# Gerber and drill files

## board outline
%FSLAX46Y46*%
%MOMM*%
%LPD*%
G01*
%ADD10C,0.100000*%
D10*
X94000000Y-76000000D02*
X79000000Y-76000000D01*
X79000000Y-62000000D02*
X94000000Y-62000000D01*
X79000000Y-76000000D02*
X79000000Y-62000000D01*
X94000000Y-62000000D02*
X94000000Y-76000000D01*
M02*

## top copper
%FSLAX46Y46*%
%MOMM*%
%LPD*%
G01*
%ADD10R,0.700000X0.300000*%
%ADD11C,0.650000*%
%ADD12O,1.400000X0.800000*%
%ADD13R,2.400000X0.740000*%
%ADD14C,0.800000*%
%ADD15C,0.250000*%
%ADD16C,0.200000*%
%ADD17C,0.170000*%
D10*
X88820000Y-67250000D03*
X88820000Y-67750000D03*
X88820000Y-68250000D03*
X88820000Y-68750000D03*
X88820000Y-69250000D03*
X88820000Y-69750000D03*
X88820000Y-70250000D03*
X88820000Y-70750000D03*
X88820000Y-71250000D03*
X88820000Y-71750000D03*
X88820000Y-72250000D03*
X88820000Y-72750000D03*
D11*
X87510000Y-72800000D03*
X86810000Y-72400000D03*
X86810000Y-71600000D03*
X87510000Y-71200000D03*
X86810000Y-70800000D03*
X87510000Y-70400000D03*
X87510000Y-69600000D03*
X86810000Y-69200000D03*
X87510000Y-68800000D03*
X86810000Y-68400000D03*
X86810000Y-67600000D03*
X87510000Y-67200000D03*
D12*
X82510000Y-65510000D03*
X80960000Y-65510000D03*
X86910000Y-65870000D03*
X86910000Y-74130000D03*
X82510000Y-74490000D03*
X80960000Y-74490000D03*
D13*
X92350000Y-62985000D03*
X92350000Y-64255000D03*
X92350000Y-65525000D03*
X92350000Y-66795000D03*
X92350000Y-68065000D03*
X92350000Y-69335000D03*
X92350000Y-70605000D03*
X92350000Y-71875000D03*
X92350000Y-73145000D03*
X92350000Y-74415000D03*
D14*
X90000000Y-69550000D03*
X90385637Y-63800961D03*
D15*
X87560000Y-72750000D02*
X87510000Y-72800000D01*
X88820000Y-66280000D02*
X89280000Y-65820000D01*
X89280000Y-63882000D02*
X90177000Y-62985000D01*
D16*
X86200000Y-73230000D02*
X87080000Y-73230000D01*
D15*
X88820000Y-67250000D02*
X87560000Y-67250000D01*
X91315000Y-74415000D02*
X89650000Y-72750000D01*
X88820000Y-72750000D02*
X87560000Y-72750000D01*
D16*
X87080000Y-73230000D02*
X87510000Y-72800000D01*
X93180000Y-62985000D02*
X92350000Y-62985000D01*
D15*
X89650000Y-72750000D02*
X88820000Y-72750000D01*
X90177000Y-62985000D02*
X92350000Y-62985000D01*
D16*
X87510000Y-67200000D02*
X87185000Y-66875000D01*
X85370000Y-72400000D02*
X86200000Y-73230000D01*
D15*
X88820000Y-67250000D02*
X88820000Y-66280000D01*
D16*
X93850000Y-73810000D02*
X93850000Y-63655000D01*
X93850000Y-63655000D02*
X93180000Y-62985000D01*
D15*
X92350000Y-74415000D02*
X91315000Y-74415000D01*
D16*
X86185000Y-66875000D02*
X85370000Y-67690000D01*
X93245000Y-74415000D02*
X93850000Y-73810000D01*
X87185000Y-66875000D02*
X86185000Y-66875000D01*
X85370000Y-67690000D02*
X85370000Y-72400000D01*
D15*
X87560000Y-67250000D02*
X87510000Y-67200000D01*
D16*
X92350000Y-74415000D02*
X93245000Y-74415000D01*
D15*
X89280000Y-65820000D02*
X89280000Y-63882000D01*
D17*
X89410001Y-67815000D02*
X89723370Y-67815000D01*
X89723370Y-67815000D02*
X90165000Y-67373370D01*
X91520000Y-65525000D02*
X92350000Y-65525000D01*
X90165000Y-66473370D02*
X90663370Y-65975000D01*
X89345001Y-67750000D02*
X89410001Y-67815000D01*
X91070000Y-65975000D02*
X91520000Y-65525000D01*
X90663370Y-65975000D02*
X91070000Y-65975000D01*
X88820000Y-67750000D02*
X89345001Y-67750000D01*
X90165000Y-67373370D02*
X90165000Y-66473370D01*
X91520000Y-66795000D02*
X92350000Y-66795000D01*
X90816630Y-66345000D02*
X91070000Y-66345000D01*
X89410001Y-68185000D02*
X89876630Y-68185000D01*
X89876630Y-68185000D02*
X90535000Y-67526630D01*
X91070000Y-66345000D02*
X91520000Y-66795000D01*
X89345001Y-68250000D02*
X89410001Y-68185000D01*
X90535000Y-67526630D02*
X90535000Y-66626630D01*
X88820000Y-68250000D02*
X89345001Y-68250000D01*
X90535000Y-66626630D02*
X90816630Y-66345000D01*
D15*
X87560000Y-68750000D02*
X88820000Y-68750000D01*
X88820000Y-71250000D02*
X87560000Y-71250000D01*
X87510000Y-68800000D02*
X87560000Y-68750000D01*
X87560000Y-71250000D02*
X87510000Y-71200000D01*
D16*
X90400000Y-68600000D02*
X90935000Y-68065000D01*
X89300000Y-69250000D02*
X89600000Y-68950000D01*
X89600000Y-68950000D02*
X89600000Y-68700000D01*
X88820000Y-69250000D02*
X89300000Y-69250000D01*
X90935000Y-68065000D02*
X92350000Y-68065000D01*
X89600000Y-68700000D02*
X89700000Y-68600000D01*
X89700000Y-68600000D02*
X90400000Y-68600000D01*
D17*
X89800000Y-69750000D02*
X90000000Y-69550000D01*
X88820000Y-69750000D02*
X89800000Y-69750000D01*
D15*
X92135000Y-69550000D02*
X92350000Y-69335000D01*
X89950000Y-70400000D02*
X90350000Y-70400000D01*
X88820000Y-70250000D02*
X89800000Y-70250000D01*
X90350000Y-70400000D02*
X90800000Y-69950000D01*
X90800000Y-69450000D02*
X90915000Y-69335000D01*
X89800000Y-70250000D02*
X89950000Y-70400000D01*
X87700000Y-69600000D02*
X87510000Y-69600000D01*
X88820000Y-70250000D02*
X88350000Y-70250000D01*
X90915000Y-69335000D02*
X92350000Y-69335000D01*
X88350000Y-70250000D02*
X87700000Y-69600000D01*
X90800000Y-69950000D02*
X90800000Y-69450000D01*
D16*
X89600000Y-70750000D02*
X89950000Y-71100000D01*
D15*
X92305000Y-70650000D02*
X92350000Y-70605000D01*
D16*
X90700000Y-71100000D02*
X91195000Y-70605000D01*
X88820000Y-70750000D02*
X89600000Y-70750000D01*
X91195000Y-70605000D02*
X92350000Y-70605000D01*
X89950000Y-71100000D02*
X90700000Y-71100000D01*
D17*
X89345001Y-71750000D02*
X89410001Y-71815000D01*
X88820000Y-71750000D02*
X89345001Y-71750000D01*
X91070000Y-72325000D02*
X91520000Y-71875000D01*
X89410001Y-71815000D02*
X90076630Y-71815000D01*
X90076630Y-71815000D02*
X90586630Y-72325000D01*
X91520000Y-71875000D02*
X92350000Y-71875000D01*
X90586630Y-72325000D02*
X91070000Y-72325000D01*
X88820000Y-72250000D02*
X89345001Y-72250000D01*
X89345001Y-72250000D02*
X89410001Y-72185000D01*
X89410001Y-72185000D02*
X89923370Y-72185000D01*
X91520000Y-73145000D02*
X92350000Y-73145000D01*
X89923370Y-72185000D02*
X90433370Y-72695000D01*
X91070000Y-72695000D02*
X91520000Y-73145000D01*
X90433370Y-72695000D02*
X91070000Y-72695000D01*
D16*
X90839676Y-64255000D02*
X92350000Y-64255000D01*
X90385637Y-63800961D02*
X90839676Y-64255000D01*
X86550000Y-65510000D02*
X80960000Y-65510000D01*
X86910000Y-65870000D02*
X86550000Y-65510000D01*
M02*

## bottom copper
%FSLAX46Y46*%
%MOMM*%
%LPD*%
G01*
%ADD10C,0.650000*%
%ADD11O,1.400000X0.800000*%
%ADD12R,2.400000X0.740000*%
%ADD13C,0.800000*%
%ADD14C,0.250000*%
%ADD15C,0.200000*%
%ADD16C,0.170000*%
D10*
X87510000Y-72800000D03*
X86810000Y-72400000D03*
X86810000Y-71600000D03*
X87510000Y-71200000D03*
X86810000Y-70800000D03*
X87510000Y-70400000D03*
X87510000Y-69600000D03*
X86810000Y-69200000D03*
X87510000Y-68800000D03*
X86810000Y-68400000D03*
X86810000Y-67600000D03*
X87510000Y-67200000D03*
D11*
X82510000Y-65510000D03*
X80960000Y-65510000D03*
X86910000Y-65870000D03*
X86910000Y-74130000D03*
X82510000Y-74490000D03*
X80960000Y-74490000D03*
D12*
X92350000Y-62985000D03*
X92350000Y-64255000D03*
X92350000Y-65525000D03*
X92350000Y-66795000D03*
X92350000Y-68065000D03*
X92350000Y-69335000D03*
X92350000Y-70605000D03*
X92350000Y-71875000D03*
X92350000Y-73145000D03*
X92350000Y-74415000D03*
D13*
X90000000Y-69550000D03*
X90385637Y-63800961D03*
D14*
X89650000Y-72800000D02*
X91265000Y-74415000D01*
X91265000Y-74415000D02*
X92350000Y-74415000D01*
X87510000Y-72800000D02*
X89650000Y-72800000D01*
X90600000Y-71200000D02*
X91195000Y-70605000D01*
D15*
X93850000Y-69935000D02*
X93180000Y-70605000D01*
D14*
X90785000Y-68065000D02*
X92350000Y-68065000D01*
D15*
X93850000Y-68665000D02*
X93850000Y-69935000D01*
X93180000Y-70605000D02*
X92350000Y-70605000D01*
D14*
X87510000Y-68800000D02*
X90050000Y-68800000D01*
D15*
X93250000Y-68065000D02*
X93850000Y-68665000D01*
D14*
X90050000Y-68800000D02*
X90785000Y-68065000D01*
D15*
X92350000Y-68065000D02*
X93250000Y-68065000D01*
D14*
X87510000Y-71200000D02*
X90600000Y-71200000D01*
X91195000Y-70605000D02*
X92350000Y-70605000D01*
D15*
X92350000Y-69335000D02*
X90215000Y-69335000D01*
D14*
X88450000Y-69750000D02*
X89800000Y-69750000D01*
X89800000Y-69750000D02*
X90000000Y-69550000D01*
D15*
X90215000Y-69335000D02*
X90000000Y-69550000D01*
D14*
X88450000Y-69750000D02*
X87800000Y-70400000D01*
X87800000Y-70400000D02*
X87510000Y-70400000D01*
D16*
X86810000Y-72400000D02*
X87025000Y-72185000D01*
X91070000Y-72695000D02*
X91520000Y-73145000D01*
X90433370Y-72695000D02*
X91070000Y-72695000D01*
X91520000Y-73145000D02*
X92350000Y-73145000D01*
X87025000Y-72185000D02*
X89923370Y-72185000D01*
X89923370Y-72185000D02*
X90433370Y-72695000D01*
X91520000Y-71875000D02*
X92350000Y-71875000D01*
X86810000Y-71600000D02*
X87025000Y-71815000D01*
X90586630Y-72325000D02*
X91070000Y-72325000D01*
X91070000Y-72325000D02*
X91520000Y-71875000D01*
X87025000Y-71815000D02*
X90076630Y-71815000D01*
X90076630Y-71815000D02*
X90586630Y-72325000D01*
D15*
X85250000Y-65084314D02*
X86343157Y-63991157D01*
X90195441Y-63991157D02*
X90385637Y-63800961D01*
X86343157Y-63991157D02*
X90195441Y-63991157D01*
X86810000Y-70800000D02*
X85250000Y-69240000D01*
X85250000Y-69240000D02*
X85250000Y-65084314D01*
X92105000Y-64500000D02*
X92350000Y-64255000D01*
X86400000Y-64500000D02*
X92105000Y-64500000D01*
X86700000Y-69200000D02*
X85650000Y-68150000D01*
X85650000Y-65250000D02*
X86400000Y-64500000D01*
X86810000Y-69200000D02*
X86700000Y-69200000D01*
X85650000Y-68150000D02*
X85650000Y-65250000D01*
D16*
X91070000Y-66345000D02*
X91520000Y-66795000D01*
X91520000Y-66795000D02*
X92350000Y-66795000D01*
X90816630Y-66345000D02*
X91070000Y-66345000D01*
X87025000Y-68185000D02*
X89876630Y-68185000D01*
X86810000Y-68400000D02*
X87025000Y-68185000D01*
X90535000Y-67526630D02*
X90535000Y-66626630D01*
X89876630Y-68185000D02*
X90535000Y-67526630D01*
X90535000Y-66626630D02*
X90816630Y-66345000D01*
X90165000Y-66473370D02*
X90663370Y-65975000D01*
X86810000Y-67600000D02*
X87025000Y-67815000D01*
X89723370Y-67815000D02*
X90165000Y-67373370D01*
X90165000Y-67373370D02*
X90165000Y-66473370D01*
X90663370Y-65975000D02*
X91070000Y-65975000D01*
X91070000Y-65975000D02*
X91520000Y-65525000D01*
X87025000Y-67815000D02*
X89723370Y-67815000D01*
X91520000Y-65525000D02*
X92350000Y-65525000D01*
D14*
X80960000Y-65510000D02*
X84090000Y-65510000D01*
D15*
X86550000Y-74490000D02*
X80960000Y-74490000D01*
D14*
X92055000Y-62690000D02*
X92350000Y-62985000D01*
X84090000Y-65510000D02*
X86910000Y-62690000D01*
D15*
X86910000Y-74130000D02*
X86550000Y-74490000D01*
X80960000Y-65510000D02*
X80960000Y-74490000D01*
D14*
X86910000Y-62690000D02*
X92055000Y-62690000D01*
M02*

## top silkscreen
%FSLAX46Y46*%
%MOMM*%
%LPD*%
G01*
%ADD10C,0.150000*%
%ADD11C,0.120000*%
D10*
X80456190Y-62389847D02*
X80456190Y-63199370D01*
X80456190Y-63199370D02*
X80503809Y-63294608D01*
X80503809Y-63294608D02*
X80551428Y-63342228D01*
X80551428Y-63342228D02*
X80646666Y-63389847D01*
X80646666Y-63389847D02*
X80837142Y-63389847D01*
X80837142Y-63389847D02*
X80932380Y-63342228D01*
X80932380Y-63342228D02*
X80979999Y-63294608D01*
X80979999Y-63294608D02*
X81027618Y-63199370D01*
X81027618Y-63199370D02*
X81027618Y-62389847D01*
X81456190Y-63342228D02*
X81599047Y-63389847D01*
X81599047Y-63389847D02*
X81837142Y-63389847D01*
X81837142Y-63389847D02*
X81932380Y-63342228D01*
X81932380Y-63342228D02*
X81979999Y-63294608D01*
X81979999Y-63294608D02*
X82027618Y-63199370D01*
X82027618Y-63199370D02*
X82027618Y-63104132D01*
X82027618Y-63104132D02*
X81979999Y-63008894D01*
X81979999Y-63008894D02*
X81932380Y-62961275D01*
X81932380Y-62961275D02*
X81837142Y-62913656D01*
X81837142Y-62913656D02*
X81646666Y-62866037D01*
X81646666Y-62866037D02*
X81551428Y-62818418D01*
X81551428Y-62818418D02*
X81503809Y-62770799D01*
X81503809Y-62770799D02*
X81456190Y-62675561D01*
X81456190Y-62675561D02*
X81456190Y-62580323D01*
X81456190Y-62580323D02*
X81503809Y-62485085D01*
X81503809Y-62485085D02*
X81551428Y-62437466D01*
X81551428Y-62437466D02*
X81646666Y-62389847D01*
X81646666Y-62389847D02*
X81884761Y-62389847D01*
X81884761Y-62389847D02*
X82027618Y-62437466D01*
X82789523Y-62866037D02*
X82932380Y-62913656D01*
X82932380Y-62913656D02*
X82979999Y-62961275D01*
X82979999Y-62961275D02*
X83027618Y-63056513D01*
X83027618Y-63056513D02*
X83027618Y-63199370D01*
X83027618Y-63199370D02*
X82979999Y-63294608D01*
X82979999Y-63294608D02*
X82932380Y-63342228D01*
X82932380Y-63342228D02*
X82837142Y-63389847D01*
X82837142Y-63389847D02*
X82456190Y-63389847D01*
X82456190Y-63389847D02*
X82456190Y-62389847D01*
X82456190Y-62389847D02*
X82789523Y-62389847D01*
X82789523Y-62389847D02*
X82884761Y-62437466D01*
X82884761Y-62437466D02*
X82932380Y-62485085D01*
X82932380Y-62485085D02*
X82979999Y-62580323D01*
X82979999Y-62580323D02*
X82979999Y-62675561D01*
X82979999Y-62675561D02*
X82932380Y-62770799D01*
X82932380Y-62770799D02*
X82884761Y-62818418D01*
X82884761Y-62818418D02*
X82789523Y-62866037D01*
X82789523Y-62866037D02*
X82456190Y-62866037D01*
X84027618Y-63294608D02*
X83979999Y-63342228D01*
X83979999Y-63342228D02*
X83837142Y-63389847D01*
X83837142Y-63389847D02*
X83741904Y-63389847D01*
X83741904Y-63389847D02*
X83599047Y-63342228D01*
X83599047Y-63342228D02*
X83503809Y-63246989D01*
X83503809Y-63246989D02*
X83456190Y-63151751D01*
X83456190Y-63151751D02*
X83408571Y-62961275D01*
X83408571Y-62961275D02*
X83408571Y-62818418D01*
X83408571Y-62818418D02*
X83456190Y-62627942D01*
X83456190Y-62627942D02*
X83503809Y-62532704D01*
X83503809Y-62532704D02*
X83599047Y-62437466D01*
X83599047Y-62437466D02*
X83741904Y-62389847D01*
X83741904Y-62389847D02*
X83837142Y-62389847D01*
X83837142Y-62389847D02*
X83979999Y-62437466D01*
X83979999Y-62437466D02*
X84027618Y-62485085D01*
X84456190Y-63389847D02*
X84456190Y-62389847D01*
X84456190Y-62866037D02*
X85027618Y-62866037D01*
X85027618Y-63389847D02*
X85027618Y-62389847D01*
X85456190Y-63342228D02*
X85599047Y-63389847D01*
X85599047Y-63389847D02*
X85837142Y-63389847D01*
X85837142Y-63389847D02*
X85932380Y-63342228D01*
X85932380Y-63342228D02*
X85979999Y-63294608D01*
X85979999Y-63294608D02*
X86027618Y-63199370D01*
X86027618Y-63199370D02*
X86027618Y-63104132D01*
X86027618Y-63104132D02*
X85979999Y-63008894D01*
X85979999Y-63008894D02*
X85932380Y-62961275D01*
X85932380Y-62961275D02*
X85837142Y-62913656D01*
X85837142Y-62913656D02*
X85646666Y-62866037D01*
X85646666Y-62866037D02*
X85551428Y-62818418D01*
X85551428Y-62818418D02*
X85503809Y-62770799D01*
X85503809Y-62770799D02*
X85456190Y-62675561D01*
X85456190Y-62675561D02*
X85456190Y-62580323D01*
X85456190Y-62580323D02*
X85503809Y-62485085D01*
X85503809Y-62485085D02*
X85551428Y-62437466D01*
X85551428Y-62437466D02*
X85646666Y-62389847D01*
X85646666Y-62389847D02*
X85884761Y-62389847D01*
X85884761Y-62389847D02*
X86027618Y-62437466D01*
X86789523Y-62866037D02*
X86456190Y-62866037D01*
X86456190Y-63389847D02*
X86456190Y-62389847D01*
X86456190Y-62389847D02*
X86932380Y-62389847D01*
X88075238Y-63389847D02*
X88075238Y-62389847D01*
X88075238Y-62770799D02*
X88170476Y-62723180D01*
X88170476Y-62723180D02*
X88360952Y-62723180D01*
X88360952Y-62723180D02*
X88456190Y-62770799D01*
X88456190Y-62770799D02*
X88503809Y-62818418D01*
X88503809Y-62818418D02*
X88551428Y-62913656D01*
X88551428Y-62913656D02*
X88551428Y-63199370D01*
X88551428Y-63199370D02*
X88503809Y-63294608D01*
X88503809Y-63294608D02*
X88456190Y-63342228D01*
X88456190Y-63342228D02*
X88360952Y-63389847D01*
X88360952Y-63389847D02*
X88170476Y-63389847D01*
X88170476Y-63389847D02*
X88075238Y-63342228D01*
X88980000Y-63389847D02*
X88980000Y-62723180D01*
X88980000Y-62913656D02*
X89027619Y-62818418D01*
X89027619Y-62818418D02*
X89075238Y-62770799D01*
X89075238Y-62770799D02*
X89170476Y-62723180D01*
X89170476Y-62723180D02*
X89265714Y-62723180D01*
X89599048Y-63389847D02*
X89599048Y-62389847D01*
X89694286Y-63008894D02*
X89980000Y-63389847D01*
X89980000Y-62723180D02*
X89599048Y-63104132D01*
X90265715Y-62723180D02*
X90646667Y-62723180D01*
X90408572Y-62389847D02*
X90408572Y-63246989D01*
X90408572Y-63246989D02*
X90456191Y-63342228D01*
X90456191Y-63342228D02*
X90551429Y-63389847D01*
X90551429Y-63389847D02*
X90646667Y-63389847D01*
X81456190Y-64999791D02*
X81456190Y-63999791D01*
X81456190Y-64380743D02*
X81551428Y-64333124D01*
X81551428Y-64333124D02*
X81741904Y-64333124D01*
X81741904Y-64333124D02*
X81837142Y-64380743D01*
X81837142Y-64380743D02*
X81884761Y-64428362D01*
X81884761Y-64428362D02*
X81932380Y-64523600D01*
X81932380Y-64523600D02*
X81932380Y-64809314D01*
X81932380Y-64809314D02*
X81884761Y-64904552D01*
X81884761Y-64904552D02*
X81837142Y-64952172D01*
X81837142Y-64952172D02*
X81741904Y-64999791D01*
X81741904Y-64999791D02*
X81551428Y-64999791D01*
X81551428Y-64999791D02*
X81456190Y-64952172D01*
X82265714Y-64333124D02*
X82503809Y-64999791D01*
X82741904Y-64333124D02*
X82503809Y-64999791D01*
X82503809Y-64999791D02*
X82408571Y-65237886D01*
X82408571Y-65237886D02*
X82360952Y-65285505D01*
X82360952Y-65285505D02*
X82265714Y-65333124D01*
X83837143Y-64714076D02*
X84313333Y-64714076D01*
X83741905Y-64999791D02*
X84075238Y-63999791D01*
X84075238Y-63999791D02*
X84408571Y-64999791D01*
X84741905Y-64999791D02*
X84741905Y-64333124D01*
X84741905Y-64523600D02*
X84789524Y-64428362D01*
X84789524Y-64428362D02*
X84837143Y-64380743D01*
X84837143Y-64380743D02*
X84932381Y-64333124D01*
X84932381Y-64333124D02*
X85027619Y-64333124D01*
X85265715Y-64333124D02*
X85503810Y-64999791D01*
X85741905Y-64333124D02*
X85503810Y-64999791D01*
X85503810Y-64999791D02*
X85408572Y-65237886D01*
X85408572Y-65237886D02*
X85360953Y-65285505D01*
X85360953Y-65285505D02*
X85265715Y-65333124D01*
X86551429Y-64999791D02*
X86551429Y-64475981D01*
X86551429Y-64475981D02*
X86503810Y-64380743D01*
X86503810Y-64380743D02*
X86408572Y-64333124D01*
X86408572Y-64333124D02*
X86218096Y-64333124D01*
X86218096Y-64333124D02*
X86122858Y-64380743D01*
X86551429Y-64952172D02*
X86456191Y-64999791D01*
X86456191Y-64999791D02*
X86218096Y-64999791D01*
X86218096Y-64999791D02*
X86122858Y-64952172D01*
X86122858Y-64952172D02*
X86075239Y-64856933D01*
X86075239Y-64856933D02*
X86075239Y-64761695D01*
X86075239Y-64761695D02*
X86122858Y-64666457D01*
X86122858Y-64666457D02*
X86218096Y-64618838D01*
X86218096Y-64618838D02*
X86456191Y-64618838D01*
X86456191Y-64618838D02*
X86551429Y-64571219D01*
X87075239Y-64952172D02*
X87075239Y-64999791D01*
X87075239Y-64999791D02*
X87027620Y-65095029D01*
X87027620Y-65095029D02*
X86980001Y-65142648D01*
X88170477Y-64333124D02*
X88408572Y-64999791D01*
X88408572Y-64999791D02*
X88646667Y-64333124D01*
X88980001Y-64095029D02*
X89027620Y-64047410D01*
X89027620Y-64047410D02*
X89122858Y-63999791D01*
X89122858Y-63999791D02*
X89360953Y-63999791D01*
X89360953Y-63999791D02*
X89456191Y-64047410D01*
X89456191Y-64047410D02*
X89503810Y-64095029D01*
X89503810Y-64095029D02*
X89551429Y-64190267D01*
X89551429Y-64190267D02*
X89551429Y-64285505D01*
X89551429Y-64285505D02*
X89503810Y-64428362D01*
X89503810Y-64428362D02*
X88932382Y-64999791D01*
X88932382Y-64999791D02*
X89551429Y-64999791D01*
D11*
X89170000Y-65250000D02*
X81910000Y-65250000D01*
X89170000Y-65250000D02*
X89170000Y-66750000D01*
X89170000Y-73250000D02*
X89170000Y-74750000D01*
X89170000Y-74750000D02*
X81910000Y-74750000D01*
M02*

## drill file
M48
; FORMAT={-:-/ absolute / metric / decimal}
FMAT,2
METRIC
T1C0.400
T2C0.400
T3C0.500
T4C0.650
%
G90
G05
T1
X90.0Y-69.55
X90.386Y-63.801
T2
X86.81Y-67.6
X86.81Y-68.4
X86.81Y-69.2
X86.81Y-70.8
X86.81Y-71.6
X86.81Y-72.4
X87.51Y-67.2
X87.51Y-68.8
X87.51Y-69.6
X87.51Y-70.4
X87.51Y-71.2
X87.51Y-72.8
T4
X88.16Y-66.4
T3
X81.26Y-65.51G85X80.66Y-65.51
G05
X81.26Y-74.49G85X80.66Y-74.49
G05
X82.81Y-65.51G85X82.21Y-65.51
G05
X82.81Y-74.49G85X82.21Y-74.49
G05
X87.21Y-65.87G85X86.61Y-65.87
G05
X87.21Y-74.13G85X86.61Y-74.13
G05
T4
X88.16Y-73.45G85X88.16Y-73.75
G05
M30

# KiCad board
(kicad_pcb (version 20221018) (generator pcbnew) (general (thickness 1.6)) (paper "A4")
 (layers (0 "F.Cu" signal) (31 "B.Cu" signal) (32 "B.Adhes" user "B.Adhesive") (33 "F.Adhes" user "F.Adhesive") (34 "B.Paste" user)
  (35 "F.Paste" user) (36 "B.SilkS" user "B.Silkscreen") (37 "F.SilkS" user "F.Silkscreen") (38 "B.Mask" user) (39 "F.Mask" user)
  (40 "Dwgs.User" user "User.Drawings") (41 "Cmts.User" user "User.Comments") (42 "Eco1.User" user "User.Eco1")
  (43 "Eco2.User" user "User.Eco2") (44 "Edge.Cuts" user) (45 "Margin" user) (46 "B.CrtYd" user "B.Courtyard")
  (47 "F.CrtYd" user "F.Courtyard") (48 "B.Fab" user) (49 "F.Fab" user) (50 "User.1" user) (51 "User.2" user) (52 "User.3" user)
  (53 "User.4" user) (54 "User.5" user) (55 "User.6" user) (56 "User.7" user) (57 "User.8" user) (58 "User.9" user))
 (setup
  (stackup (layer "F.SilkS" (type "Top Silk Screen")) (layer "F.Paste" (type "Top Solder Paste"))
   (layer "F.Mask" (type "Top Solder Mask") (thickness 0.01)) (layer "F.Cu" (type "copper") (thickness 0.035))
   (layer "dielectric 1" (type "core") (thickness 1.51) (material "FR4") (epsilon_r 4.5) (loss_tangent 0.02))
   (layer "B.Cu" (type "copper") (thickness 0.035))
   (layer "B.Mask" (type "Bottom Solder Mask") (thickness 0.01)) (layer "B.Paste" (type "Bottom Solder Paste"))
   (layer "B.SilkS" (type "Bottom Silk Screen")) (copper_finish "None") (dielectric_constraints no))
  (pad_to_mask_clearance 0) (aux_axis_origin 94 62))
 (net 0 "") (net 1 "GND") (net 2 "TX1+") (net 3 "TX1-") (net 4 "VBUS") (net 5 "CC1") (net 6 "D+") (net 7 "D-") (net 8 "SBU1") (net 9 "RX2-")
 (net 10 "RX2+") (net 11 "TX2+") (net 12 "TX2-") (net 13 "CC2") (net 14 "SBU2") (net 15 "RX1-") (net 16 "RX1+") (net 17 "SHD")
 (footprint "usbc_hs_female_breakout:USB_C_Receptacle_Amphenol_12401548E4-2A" (layer "F.Cu") (at 83.8 70 -90)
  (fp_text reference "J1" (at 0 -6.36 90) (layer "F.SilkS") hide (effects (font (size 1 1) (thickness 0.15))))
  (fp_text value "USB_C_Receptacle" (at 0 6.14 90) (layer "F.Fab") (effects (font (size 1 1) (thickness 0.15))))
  (fp_line (start -4.75 -5.37) (end -4.75 1.89) (stroke (width 0.12) (type solid)) (layer "F.SilkS"))
  (fp_line (start -4.75 -5.37) (end -3.25 -5.37) (stroke (width 0.12) (type solid)) (layer "F.SilkS"))
  (fp_line (start 3.25 -5.37) (end 4.75 -5.37) (stroke (width 0.12) (type solid)) (layer "F.SilkS"))
  (fp_line (start 4.75 -5.37) (end 4.75 1.89) (stroke (width 0.12) (type solid)) (layer "F.SilkS"))
  (pad "" np_thru_hole circle (at -3.6 -4.36 270) (size 0.65 0.65) (drill 0.65) (layers "*.Cu" "*.Mask"))
  (pad "" np_thru_hole oval (at 3.6 -4.36 270) (size 0.95 0.65) (drill oval 0.95 0.65) (layers "*.Cu" "*.Mask"))
  (pad "A1" smd rect (at -2.75 -5.02 270) (size 0.3 0.7) (layers "F.Cu" "F.Paste" "F.Mask") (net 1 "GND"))
  (pad "A2" smd rect (at -2.25 -5.02 270) (size 0.3 0.7) (layers "F.Cu" "F.Paste" "F.Mask") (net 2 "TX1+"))
  (pad "A3" smd rect (at -1.75 -5.02 270) (size 0.3 0.7) (layers "F.Cu" "F.Paste" "F.Mask") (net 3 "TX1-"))
  (pad "A4" smd rect (at -1.25 -5.02 270) (size 0.3 0.7) (layers "F.Cu" "F.Paste" "F.Mask") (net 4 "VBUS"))
  (pad "A5" smd rect (at -0.75 -5.02 270) (size 0.3 0.7) (layers "F.Cu" "F.Paste" "F.Mask") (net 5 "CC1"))
  (pad "A6" smd rect (at -0.25 -5.02 270) (size 0.3 0.7) (layers "F.Cu" "F.Paste" "F.Mask") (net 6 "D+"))
  (pad "A7" smd rect (at 0.25 -5.02 270) (size 0.3 0.7) (layers "F.Cu" "F.Paste" "F.Mask") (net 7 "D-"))
  (pad "A8" smd rect (at 0.75 -5.02 270) (size 0.3 0.7) (layers "F.Cu" "F.Paste" "F.Mask") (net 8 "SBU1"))
  (pad "A9" smd rect (at 1.25 -5.02 270) (size 0.3 0.7) (layers "F.Cu" "F.Paste" "F.Mask") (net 4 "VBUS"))
  (pad "A10" smd rect (at 1.75 -5.02 270) (size 0.3 0.7) (layers "F.Cu" "F.Paste" "F.Mask") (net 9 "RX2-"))
  (pad "A11" smd rect (at 2.25 -5.02 270) (size 0.3 0.7) (layers "F.Cu" "F.Paste" "F.Mask") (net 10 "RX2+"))
  (pad "A12" smd rect (at 2.75 -5.02 270) (size 0.3 0.7) (layers "F.Cu" "F.Paste" "F.Mask") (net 1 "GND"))
  (pad "B1" thru_hole circle (at 2.8 -3.71 270) (size 0.65 0.65) (drill 0.4) (layers "*.Cu" "*.Mask") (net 1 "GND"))
  (pad "B2" thru_hole circle (at 2.4 -3.01 270) (size 0.65 0.65) (drill 0.4) (layers "*.Cu" "*.Mask") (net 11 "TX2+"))
  (pad "B3" thru_hole circle (at 1.6 -3.01 270) (size 0.65 0.65) (drill 0.4) (layers "*.Cu" "*.Mask") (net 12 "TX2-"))
  (pad "B4" thru_hole circle (at 1.2 -3.71 270) (size 0.65 0.65) (drill 0.4) (layers "*.Cu" "*.Mask") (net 4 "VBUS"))
  (pad "B5" thru_hole circle (at 0.8 -3.01 270) (size 0.65 0.65) (drill 0.4) (layers "*.Cu" "*.Mask") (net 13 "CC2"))
  (pad "B6" thru_hole circle (at 0.4 -3.71 270) (size 0.65 0.65) (drill 0.4) (layers "*.Cu" "*.Mask") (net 6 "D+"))
  (pad "B7" thru_hole circle (at -0.4 -3.71 270) (size 0.65 0.65) (drill 0.4) (layers "*.Cu" "*.Mask") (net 7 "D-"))
  (pad "B8" thru_hole circle (at -0.8 -3.01 270) (size 0.65 0.65) (drill 0.4) (layers "*.Cu" "*.Mask") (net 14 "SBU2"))
  (pad "B9" thru_hole circle (at -1.2 -3.71 270) (size 0.65 0.65) (drill 0.4) (layers "*.Cu" "*.Mask") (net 4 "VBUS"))
  (pad "B10" thru_hole circle (at -1.6 -3.01 270) (size 0.65 0.65) (drill 0.4) (layers "*.Cu" "*.Mask") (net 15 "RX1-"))
  (pad "B11" thru_hole circle (at -2.4 -3.01 270) (size 0.65 0.65) (drill 0.4) (layers "*.Cu" "*.Mask") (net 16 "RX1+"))
  (pad "B12" thru_hole circle (at -2.8 -3.71 270) (size 0.65 0.65) (drill 0.4) (layers "*.Cu" "*.Mask") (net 1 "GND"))
  (pad "S1" thru_hole oval (at -4.49 1.29 270) (size 0.8 1.4) (drill oval 0.5 1.1) (layers "*.Cu" "*.Mask") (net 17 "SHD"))
  (pad "S1" thru_hole oval (at -4.49 2.84 270) (size 0.8 1.4) (drill oval 0.5 1.1) (layers "*.Cu" "*.Mask") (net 17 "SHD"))
  (pad "S1" thru_hole oval (at -4.13 -3.11 270) (size 0.8 1.4) (drill oval 0.5 1.1) (layers "*.Cu" "*.Mask") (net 17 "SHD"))
  (pad "S1" thru_hole oval (at 4.13 -3.11 270) (size 0.8 1.4) (drill oval 0.5 1.1) (layers "*.Cu" "*.Mask") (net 17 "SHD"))
  (pad "S1" thru_hole oval (at 4.49 1.29 270) (size 0.8 1.4) (drill oval 0.5 1.1) (layers "*.Cu" "*.Mask") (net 17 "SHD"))
  (pad "S1" thru_hole oval (at 4.49 2.84 270) (size 0.8 1.4) (drill oval 0.5 1.1) (layers "*.Cu" "*.Mask") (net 17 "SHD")))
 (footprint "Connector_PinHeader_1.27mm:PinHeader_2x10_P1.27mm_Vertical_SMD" (layer "F.Cu") (at 92.468 68.7)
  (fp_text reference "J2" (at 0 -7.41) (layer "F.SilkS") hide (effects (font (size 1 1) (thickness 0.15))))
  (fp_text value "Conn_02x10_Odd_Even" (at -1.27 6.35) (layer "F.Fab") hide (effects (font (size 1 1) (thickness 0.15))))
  (pad "1" smd rect (at -0.118 -5.715) (size 2.4 0.74) (layers "F.Cu" "F.Mask") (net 1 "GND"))
  (pad "2" smd rect (at -0.118 -5.715) (size 2.4 0.74) (layers "B.Cu" "B.Paste" "B.Mask") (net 17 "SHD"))
  (pad "3" smd rect (at -0.118 -4.445) (size 2.4 0.74) (layers "F.Cu" "F.Mask") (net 13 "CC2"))
  (pad "4" smd rect (at -0.118 -4.445) (size 2.4 0.74) (layers "B.Cu" "B.Paste" "B.Mask") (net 14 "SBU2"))
  (pad "5" smd rect (at -0.118 -3.175) (size 2.4 0.74) (layers "F.Cu" "F.Mask") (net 2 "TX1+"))
  (pad "6" smd rect (at -0.118 -3.175) (size 2.4 0.74) (layers "B.Cu" "B.Paste" "B.Mask") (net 16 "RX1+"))
  (pad "7" smd rect (at -0.118 -1.905) (size 2.4 0.74) (layers "F.Cu" "F.Mask") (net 3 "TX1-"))
  (pad "8" smd rect (at -0.118 -1.905) (size 2.4 0.74) (layers "B.Cu" "B.Paste" "B.Mask") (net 15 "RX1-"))
  (pad "9" smd rect (at -0.118 -0.635) (size 2.4 0.74) (layers "F.Cu" "F.Mask") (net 5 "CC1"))
  (pad "10" smd rect (at -0.118 -0.635) (size 2.4 0.74) (layers "B.Cu" "B.Paste" "B.Mask") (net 4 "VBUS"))
  (pad "11" smd rect (at -0.118 0.635) (size 2.4 0.74) (layers "F.Cu" "F.Mask") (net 7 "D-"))
  (pad "12" smd rect (at -0.118 0.635) (size 2.4 0.74) (layers "B.Cu" "B.Paste" "B.Mask") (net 6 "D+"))
  (pad "13" smd rect (at -0.118 1.905) (size 2.4 0.74) (layers "F.Cu" "F.Mask") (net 8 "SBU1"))
  (pad "14" smd rect (at -0.118 1.905) (size 2.4 0.74) (layers "B.Cu" "B.Paste" "B.Mask") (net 4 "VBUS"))
  (pad "15" smd rect (at -0.118 3.175) (size 2.4 0.74) (layers "F.Cu" "F.Mask") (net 9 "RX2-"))
  (pad "16" smd rect (at -0.118 3.175) (size 2.4 0.74) (layers "B.Cu" "B.Paste" "B.Mask") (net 12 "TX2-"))
  (pad "17" smd rect (at -0.118 4.445) (size 2.4 0.74) (layers "F.Cu" "F.Mask") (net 10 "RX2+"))
  (pad "18" smd rect (at -0.118 4.445) (size 2.4 0.74) (layers "B.Cu" "B.Paste" "B.Mask") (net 11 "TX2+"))
  (pad "19" smd rect (at -0.118 5.715) (size 2.4 0.74) (layers "F.Cu" "F.Mask") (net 1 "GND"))
  (pad "20" smd rect (at -0.118 5.715) (size 2.4 0.74) (layers "B.Cu" "B.Paste" "B.Mask") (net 1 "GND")))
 (gr_line (start 94 76) (end 79 76) (stroke (width 0.1) (type solid)) (layer "Edge.Cuts"))
 (gr_line (start 79 62) (end 94 62) (stroke (width 0.1) (type solid)) (layer "Edge.Cuts"))
 (gr_line (start 79 76) (end 79 62) (stroke (width 0.1) (type solid)) (layer "Edge.Cuts"))
 (gr_line (start 94 62) (end 94 76) (stroke (width 0.1) (type solid)) (layer "Edge.Cuts"))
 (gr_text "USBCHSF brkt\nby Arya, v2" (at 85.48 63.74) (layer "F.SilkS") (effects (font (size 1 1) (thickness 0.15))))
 (segment (start 87.56 72.75) (end 87.51 72.8) (width 0.25) (layer "F.Cu") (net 1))
 (segment (start 88.82 66.28) (end 89.28 65.82) (width 0.25) (layer "F.Cu") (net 1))
 (segment (start 89.28 63.882) (end 90.177 62.985) (width 0.25) (layer "F.Cu") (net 1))
 (segment (start 86.2 73.23) (end 87.08 73.23) (width 0.2) (layer "F.Cu") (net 1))
 (segment (start 88.82 67.25) (end 87.56 67.25) (width 0.25) (layer "F.Cu") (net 1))
 (segment (start 91.315 74.415) (end 89.65 72.75) (width 0.25) (layer "F.Cu") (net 1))
 (segment (start 88.82 72.75) (end 87.56 72.75) (width 0.25) (layer "F.Cu") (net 1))
 (segment (start 87.08 73.23) (end 87.51 72.8) (width 0.2) (layer "F.Cu") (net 1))
 (segment (start 93.18 62.985) (end 92.35 62.985) (width 0.2) (layer "F.Cu") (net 1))
 (segment (start 89.65 72.75) (end 88.82 72.75) (width 0.25) (layer "F.Cu") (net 1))
 (segment (start 90.177 62.985) (end 92.35 62.985) (width 0.25) (layer "F.Cu") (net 1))
 (segment (start 87.51 67.2) (end 87.185 66.875) (width 0.2) (layer "F.Cu") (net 1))
 (segment (start 85.37 72.4) (end 86.2 73.23) (width 0.2) (layer "F.Cu") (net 1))
 (segment (start 88.82 67.25) (end 88.82 66.28) (width 0.25) (layer "F.Cu") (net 1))
 (segment (start 93.85 73.81) (end 93.85 63.655) (width 0.2) (layer "F.Cu") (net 1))
 (segment (start 93.85 63.655) (end 93.18 62.985) (width 0.2) (layer "F.Cu") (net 1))
 (segment (start 92.35 74.415) (end 91.315 74.415) (width 0.25) (layer "F.Cu") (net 1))
 (segment (start 86.185 66.875) (end 85.37 67.69) (width 0.2) (layer "F.Cu") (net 1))
 (segment (start 93.245 74.415) (end 93.85 73.81) (width 0.2) (layer "F.Cu") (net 1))
 (segment (start 87.185 66.875) (end 86.185 66.875) (width 0.2) (layer "F.Cu") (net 1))
 (segment (start 85.37 67.69) (end 85.37 72.4) (width 0.2) (layer "F.Cu") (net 1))
 (segment (start 87.56 67.25) (end 87.51 67.2) (width 0.25) (layer "F.Cu") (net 1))
 (segment (start 92.35 74.415) (end 93.245 74.415) (width 0.2) (layer "F.Cu") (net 1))
 (segment (start 89.28 65.82) (end 89.28 63.882) (width 0.25) (layer "F.Cu") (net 1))
 (segment (start 89.65 72.8) (end 91.265 74.415) (width 0.25) (layer "B.Cu") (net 1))
 (segment (start 91.265 74.415) (end 92.35 74.415) (width 0.25) (layer "B.Cu") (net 1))
 (segment (start 87.51 72.8) (end 89.65 72.8) (width 0.25) (layer "B.Cu") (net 1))
 (segment (start 89.410001 67.815) (end 89.72337 67.815) (width 0.17) (layer "F.Cu") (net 2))
 (segment (start 89.72337 67.815) (end 90.165 67.37337) (width 0.17) (layer "F.Cu") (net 2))
 (segment (start 91.52 65.525) (end 92.35 65.525) (width 0.17) (layer "F.Cu") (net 2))
 (segment (start 90.165 66.47337) (end 90.66337 65.975) (width 0.17) (layer "F.Cu") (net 2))
 (segment (start 89.345001 67.75) (end 89.410001 67.815) (width 0.17) (layer "F.Cu") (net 2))
 (segment (start 91.07 65.975) (end 91.52 65.525) (width 0.17) (layer "F.Cu") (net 2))
 (segment (start 90.66337 65.975) (end 91.07 65.975) (width 0.17) (layer "F.Cu") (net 2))
 (segment (start 88.82 67.75) (end 89.345001 67.75) (width 0.17) (layer "F.Cu") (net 2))
 (segment (start 90.165 67.37337) (end 90.165 66.47337) (width 0.17) (layer "F.Cu") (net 2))
 (segment (start 91.52 66.795) (end 92.35 66.795) (width 0.17) (layer "F.Cu") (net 3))
 (segment (start 90.81663 66.345) (end 91.07 66.345) (width 0.17) (layer "F.Cu") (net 3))
 (segment (start 89.410001 68.185) (end 89.87663 68.185) (width 0.17) (layer "F.Cu") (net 3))
 (segment (start 89.87663 68.185) (end 90.535 67.52663) (width 0.17) (layer "F.Cu") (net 3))
 (segment (start 91.07 66.345) (end 91.52 66.795) (width 0.17) (layer "F.Cu") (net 3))
 (segment (start 89.345001 68.25) (end 89.410001 68.185) (width 0.17) (layer "F.Cu") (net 3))
 (segment (start 90.535 67.52663) (end 90.535 66.62663) (width 0.17) (layer "F.Cu") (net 3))
 (segment (start 88.82 68.25) (end 89.345001 68.25) (width 0.17) (layer "F.Cu") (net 3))
 (segment (start 90.535 66.62663) (end 90.81663 66.345) (width 0.17) (layer "F.Cu") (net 3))
 (segment (start 87.56 68.75) (end 88.82 68.75) (width 0.25) (layer "F.Cu") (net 4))
 (segment (start 88.82 71.25) (end 87.56 71.25) (width 0.25) (layer "F.Cu") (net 4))
 (segment (start 87.51 68.8) (end 87.56 68.75) (width 0.25) (layer "F.Cu") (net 4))
 (segment (start 87.56 71.25) (end 87.51 71.2) (width 0.25) (layer "F.Cu") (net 4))
 (segment (start 90.6 71.2) (end 91.195 70.605) (width 0.25) (layer "B.Cu") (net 4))
 (segment (start 93.85 69.935) (end 93.18 70.605) (width 0.2) (layer "B.Cu") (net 4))
 (segment (start 90.785 68.065) (end 92.35 68.065) (width 0.25) (layer "B.Cu") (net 4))
 (segment (start 93.85 68.665) (end 93.85 69.935) (width 0.2) (layer "B.Cu") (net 4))
 (segment (start 93.18 70.605) (end 92.35 70.605) (width 0.2) (layer "B.Cu") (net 4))
 (segment (start 87.51 68.8) (end 90.05 68.8) (width 0.25) (layer "B.Cu") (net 4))
 (segment (start 93.25 68.065) (end 93.85 68.665) (width 0.2) (layer "B.Cu") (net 4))
 (segment (start 90.05 68.8) (end 90.785 68.065) (width 0.25) (layer "B.Cu") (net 4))
 (segment (start 92.35 68.065) (end 93.25 68.065) (width 0.2) (layer "B.Cu") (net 4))
 (segment (start 87.51 71.2) (end 90.6 71.2) (width 0.25) (layer "B.Cu") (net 4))
 (segment (start 91.195 70.605) (end 92.35 70.605) (width 0.25) (layer "B.Cu") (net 4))
 (segment (start 90.4 68.6) (end 90.935 68.065) (width 0.2) (layer "F.Cu") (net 5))
 (segment (start 89.3 69.25) (end 89.6 68.95) (width 0.2) (layer "F.Cu") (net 5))
 (segment (start 89.6 68.95) (end 89.6 68.7) (width 0.2) (layer "F.Cu") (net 5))
 (segment (start 88.82 69.25) (end 89.3 69.25) (width 0.2) (layer "F.Cu") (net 5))
 (segment (start 90.935 68.065) (end 92.35 68.065) (width 0.2) (layer "F.Cu") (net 5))
 (segment (start 89.6 68.7) (end 89.7 68.6) (width 0.2) (layer "F.Cu") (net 5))
 (segment (start 89.7 68.6) (end 90.4 68.6) (width 0.2) (layer "F.Cu") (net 5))
 (segment (start 89.8 69.75) (end 90 69.55) (width 0.17) (layer "F.Cu") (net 6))
 (segment (start 88.82 69.75) (end 89.8 69.75) (width 0.17) (layer "F.Cu") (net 6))
 (via (at 90 69.55) (size 0.8) (drill 0.4) (layers "F.Cu" "B.Cu") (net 6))
 (segment (start 92.35 69.335) (end 90.215 69.335) (width 0.2) (layer "B.Cu") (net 6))
 (segment (start 88.45 69.75) (end 89.8 69.75) (width 0.25) (layer "B.Cu") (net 6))
 (segment (start 89.8 69.75) (end 90 69.55) (width 0.25) (layer "B.Cu") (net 6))
 (segment (start 90.215 69.335) (end 90 69.55) (width 0.2) (layer "B.Cu") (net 6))
 (segment (start 88.45 69.75) (end 87.8 70.4) (width 0.25) (layer "B.Cu") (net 6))
 (segment (start 87.8 70.4) (end 87.51 70.4) (width 0.25) (layer "B.Cu") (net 6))
 (segment (start 92.135 69.55) (end 92.35 69.335) (width 0.25) (layer "F.Cu") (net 7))
 (segment (start 89.95 70.4) (end 90.35 70.4) (width 0.25) (layer "F.Cu") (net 7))
 (segment (start 88.82 70.25) (end 89.8 70.25) (width 0.25) (layer "F.Cu") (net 7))
 (segment (start 90.35 70.4) (end 90.8 69.95) (width 0.25) (layer "F.Cu") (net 7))
 (segment (start 90.8 69.45) (end 90.915 69.335) (width 0.25) (layer "F.Cu") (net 7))
 (segment (start 89.8 70.25) (end 89.95 70.4) (width 0.25) (layer "F.Cu") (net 7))
 (segment (start 87.7 69.6) (end 87.51 69.6) (width 0.25) (layer "F.Cu") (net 7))
 (segment (start 88.82 70.25) (end 88.35 70.25) (width 0.25) (layer "F.Cu") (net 7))
 (segment (start 90.915 69.335) (end 92.35 69.335) (width 0.25) (layer "F.Cu") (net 7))
 (segment (start 88.35 70.25) (end 87.7 69.6) (width 0.25) (layer "F.Cu") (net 7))
 (segment (start 90.8 69.95) (end 90.8 69.45) (width 0.25) (layer "F.Cu") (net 7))
 (segment (start 89.6 70.75) (end 89.95 71.1) (width 0.2) (layer "F.Cu") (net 8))
 (segment (start 92.305 70.65) (end 92.35 70.605) (width 0.25) (layer "F.Cu") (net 8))
 (segment (start 90.7 71.1) (end 91.195 70.605) (width 0.2) (layer "F.Cu") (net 8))
 (segment (start 88.82 70.75) (end 89.6 70.75) (width 0.2) (layer "F.Cu") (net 8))
 (segment (start 91.195 70.605) (end 92.35 70.605) (width 0.2) (layer "F.Cu") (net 8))
 (segment (start 89.95 71.1) (end 90.7 71.1) (width 0.2) (layer "F.Cu") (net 8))
 (segment (start 89.345001 71.75) (end 89.410001 71.815) (width 0.17) (layer "F.Cu") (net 9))
 (segment (start 88.82 71.75) (end 89.345001 71.75) (width 0.17) (layer "F.Cu") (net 9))
 (segment (start 91.07 72.325) (end 91.52 71.875) (width 0.17) (layer "F.Cu") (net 9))
 (segment (start 89.410001 71.815) (end 90.07663 71.815) (width 0.17) (layer "F.Cu") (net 9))
 (segment (start 90.07663 71.815) (end 90.58663 72.325) (width 0.17) (layer "F.Cu") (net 9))
 (segment (start 91.52 71.875) (end 92.35 71.875) (width 0.17) (layer "F.Cu") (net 9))
 (segment (start 90.58663 72.325) (end 91.07 72.325) (width 0.17) (layer "F.Cu") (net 9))
 (segment (start 88.82 72.25) (end 89.345001 72.25) (width 0.17) (layer "F.Cu") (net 10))
 (segment (start 89.345001 72.25) (end 89.410001 72.185) (width 0.17) (layer "F.Cu") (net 10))
 (segment (start 89.410001 72.185) (end 89.92337 72.185) (width 0.17) (layer "F.Cu") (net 10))
 (segment (start 91.52 73.145) (end 92.35 73.145) (width 0.17) (layer "F.Cu") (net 10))
 (segment (start 89.92337 72.185) (end 90.43337 72.695) (width 0.17) (layer "F.Cu") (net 10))
 (segment (start 91.07 72.695) (end 91.52 73.145) (width 0.17) (layer "F.Cu") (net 10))
 (segment (start 90.43337 72.695) (end 91.07 72.695) (width 0.17) (layer "F.Cu") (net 10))
 (segment (start 86.81 72.4) (end 87.025 72.185) (width 0.17) (layer "B.Cu") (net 11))
 (segment (start 91.07 72.695) (end 91.52 73.145) (width 0.17) (layer "B.Cu") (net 11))
 (segment (start 90.43337 72.695) (end 91.07 72.695) (width 0.17) (layer "B.Cu") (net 11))
 (segment (start 91.52 73.145) (end 92.35 73.145) (width 0.17) (layer "B.Cu") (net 11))
 (segment (start 87.025 72.185) (end 89.92337 72.185) (width 0.17) (layer "B.Cu") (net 11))
 (segment (start 89.92337 72.185) (end 90.43337 72.695) (width 0.17) (layer "B.Cu") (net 11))
 (segment (start 91.52 71.875) (end 92.35 71.875) (width 0.17) (layer "B.Cu") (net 12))
 (segment (start 86.81 71.6) (end 87.025 71.815) (width 0.17) (layer "B.Cu") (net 12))
 (segment (start 90.58663 72.325) (end 91.07 72.325) (width 0.17) (layer "B.Cu") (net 12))
 (segment (start 91.07 72.325) (end 91.52 71.875) (width 0.17) (layer "B.Cu") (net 12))
 (segment (start 87.025 71.815) (end 90.07663 71.815) (width 0.17) (layer "B.Cu") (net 12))
 (segment (start 90.07663 71.815) (end 90.58663 72.325) (width 0.17) (layer "B.Cu") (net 12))
 (segment (start 90.839676 64.255) (end 92.35 64.255) (width 0.2) (layer "F.Cu") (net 13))
 (segment (start 90.385637 63.800961) (end 90.839676 64.255) (width 0.2) (layer "F.Cu") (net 13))
 (via (at 90.385637 63.800961) (size 0.8) (drill 0.4) (layers "F.Cu" "B.Cu") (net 13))
 (segment (start 85.25 65.084314) (end 86.343157 63.991157) (width 0.2) (layer "B.Cu") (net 13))
 (segment (start 90.195441 63.991157) (end 90.385637 63.800961) (width 0.2) (layer "B.Cu") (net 13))
 (segment (start 86.343157 63.991157) (end 90.195441 63.991157) (width 0.2) (layer "B.Cu") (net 13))
 (segment (start 86.81 70.8) (end 85.25 69.24) (width 0.2) (layer "B.Cu") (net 13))
 (segment (start 85.25 69.24) (end 85.25 65.084314) (width 0.2) (layer "B.Cu") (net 13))
 (segment (start 92.105 64.5) (end 92.35 64.255) (width 0.2) (layer "B.Cu") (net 14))
 (segment (start 86.4 64.5) (end 92.105 64.5) (width 0.2) (layer "B.Cu") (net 14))
 (segment (start 86.7 69.2) (end 85.65 68.15) (width 0.2) (layer "B.Cu") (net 14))
 (segment (start 85.65 65.25) (end 86.4 64.5) (width 0.2) (layer "B.Cu") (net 14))
 (segment (start 86.81 69.2) (end 86.7 69.2) (width 0.2) (layer "B.Cu") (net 14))
 (segment (start 85.65 68.15) (end 85.65 65.25) (width 0.2) (layer "B.Cu") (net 14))
 (segment (start 91.07 66.345) (end 91.52 66.795) (width 0.17) (layer "B.Cu") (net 15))
 (segment (start 91.52 66.795) (end 92.35 66.795) (width 0.17) (layer "B.Cu") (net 15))
 (segment (start 90.81663 66.345) (end 91.07 66.345) (width 0.17) (layer "B.Cu") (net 15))
 (segment (start 87.025 68.185) (end 89.87663 68.185) (width 0.17) (layer "B.Cu") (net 15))
 (segment (start 86.81 68.4) (end 87.025 68.185) (width 0.17) (layer "B.Cu") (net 15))
 (segment (start 90.535 67.52663) (end 90.535 66.62663) (width 0.17) (layer "B.Cu") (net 15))
 (segment (start 89.87663 68.185) (end 90.535 67.52663) (width 0.17) (layer "B.Cu") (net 15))
 (segment (start 90.535 66.62663) (end 90.81663 66.345) (width 0.17) (layer "B.Cu") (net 15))
 (segment (start 90.165 66.47337) (end 90.66337 65.975) (width 0.17) (layer "B.Cu") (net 16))
 (segment (start 86.81 67.6) (end 87.025 67.815) (width 0.17) (layer "B.Cu") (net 16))
 (segment (start 89.72337 67.815) (end 90.165 67.37337) (width 0.17) (layer "B.Cu") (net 16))
 (segment (start 90.165 67.37337) (end 90.165 66.47337) (width 0.17) (layer "B.Cu") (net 16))
 (segment (start 90.66337 65.975) (end 91.07 65.975) (width 0.17) (layer "B.Cu") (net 16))
 (segment (start 91.07 65.975) (end 91.52 65.525) (width 0.17) (layer "B.Cu") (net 16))
 (segment (start 87.025 67.815) (end 89.72337 67.815) (width 0.17) (layer "B.Cu") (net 16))
 (segment (start 91.52 65.525) (end 92.35 65.525) (width 0.17) (layer "B.Cu") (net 16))
 (segment (start 86.55 65.51) (end 80.96 65.51) (width 0.2) (layer "F.Cu") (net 17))
 (segment (start 86.91 65.87) (end 86.55 65.51) (width 0.2) (layer "F.Cu") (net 17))
 (segment (start 80.96 65.51) (end 84.09 65.51) (width 0.25) (layer "B.Cu") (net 17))
 (segment (start 86.55 74.49) (end 80.96 74.49) (width 0.2) (layer "B.Cu") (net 17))
 (segment (start 92.055 62.69) (end 92.35 62.985) (width 0.25) (layer "B.Cu") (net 17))
 (segment (start 84.09 65.51) (end 86.91 62.69) (width 0.25) (layer "B.Cu") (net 17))
 (segment (start 86.91 74.13) (end 86.55 74.49) (width 0.2) (layer "B.Cu") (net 17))
 (segment (start 80.96 65.51) (end 80.96 74.49) (width 0.2) (layer "B.Cu") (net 17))
 (segment (start 86.91 62.69) (end 92.055 62.69) (width 0.25) (layer "B.Cu") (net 17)))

